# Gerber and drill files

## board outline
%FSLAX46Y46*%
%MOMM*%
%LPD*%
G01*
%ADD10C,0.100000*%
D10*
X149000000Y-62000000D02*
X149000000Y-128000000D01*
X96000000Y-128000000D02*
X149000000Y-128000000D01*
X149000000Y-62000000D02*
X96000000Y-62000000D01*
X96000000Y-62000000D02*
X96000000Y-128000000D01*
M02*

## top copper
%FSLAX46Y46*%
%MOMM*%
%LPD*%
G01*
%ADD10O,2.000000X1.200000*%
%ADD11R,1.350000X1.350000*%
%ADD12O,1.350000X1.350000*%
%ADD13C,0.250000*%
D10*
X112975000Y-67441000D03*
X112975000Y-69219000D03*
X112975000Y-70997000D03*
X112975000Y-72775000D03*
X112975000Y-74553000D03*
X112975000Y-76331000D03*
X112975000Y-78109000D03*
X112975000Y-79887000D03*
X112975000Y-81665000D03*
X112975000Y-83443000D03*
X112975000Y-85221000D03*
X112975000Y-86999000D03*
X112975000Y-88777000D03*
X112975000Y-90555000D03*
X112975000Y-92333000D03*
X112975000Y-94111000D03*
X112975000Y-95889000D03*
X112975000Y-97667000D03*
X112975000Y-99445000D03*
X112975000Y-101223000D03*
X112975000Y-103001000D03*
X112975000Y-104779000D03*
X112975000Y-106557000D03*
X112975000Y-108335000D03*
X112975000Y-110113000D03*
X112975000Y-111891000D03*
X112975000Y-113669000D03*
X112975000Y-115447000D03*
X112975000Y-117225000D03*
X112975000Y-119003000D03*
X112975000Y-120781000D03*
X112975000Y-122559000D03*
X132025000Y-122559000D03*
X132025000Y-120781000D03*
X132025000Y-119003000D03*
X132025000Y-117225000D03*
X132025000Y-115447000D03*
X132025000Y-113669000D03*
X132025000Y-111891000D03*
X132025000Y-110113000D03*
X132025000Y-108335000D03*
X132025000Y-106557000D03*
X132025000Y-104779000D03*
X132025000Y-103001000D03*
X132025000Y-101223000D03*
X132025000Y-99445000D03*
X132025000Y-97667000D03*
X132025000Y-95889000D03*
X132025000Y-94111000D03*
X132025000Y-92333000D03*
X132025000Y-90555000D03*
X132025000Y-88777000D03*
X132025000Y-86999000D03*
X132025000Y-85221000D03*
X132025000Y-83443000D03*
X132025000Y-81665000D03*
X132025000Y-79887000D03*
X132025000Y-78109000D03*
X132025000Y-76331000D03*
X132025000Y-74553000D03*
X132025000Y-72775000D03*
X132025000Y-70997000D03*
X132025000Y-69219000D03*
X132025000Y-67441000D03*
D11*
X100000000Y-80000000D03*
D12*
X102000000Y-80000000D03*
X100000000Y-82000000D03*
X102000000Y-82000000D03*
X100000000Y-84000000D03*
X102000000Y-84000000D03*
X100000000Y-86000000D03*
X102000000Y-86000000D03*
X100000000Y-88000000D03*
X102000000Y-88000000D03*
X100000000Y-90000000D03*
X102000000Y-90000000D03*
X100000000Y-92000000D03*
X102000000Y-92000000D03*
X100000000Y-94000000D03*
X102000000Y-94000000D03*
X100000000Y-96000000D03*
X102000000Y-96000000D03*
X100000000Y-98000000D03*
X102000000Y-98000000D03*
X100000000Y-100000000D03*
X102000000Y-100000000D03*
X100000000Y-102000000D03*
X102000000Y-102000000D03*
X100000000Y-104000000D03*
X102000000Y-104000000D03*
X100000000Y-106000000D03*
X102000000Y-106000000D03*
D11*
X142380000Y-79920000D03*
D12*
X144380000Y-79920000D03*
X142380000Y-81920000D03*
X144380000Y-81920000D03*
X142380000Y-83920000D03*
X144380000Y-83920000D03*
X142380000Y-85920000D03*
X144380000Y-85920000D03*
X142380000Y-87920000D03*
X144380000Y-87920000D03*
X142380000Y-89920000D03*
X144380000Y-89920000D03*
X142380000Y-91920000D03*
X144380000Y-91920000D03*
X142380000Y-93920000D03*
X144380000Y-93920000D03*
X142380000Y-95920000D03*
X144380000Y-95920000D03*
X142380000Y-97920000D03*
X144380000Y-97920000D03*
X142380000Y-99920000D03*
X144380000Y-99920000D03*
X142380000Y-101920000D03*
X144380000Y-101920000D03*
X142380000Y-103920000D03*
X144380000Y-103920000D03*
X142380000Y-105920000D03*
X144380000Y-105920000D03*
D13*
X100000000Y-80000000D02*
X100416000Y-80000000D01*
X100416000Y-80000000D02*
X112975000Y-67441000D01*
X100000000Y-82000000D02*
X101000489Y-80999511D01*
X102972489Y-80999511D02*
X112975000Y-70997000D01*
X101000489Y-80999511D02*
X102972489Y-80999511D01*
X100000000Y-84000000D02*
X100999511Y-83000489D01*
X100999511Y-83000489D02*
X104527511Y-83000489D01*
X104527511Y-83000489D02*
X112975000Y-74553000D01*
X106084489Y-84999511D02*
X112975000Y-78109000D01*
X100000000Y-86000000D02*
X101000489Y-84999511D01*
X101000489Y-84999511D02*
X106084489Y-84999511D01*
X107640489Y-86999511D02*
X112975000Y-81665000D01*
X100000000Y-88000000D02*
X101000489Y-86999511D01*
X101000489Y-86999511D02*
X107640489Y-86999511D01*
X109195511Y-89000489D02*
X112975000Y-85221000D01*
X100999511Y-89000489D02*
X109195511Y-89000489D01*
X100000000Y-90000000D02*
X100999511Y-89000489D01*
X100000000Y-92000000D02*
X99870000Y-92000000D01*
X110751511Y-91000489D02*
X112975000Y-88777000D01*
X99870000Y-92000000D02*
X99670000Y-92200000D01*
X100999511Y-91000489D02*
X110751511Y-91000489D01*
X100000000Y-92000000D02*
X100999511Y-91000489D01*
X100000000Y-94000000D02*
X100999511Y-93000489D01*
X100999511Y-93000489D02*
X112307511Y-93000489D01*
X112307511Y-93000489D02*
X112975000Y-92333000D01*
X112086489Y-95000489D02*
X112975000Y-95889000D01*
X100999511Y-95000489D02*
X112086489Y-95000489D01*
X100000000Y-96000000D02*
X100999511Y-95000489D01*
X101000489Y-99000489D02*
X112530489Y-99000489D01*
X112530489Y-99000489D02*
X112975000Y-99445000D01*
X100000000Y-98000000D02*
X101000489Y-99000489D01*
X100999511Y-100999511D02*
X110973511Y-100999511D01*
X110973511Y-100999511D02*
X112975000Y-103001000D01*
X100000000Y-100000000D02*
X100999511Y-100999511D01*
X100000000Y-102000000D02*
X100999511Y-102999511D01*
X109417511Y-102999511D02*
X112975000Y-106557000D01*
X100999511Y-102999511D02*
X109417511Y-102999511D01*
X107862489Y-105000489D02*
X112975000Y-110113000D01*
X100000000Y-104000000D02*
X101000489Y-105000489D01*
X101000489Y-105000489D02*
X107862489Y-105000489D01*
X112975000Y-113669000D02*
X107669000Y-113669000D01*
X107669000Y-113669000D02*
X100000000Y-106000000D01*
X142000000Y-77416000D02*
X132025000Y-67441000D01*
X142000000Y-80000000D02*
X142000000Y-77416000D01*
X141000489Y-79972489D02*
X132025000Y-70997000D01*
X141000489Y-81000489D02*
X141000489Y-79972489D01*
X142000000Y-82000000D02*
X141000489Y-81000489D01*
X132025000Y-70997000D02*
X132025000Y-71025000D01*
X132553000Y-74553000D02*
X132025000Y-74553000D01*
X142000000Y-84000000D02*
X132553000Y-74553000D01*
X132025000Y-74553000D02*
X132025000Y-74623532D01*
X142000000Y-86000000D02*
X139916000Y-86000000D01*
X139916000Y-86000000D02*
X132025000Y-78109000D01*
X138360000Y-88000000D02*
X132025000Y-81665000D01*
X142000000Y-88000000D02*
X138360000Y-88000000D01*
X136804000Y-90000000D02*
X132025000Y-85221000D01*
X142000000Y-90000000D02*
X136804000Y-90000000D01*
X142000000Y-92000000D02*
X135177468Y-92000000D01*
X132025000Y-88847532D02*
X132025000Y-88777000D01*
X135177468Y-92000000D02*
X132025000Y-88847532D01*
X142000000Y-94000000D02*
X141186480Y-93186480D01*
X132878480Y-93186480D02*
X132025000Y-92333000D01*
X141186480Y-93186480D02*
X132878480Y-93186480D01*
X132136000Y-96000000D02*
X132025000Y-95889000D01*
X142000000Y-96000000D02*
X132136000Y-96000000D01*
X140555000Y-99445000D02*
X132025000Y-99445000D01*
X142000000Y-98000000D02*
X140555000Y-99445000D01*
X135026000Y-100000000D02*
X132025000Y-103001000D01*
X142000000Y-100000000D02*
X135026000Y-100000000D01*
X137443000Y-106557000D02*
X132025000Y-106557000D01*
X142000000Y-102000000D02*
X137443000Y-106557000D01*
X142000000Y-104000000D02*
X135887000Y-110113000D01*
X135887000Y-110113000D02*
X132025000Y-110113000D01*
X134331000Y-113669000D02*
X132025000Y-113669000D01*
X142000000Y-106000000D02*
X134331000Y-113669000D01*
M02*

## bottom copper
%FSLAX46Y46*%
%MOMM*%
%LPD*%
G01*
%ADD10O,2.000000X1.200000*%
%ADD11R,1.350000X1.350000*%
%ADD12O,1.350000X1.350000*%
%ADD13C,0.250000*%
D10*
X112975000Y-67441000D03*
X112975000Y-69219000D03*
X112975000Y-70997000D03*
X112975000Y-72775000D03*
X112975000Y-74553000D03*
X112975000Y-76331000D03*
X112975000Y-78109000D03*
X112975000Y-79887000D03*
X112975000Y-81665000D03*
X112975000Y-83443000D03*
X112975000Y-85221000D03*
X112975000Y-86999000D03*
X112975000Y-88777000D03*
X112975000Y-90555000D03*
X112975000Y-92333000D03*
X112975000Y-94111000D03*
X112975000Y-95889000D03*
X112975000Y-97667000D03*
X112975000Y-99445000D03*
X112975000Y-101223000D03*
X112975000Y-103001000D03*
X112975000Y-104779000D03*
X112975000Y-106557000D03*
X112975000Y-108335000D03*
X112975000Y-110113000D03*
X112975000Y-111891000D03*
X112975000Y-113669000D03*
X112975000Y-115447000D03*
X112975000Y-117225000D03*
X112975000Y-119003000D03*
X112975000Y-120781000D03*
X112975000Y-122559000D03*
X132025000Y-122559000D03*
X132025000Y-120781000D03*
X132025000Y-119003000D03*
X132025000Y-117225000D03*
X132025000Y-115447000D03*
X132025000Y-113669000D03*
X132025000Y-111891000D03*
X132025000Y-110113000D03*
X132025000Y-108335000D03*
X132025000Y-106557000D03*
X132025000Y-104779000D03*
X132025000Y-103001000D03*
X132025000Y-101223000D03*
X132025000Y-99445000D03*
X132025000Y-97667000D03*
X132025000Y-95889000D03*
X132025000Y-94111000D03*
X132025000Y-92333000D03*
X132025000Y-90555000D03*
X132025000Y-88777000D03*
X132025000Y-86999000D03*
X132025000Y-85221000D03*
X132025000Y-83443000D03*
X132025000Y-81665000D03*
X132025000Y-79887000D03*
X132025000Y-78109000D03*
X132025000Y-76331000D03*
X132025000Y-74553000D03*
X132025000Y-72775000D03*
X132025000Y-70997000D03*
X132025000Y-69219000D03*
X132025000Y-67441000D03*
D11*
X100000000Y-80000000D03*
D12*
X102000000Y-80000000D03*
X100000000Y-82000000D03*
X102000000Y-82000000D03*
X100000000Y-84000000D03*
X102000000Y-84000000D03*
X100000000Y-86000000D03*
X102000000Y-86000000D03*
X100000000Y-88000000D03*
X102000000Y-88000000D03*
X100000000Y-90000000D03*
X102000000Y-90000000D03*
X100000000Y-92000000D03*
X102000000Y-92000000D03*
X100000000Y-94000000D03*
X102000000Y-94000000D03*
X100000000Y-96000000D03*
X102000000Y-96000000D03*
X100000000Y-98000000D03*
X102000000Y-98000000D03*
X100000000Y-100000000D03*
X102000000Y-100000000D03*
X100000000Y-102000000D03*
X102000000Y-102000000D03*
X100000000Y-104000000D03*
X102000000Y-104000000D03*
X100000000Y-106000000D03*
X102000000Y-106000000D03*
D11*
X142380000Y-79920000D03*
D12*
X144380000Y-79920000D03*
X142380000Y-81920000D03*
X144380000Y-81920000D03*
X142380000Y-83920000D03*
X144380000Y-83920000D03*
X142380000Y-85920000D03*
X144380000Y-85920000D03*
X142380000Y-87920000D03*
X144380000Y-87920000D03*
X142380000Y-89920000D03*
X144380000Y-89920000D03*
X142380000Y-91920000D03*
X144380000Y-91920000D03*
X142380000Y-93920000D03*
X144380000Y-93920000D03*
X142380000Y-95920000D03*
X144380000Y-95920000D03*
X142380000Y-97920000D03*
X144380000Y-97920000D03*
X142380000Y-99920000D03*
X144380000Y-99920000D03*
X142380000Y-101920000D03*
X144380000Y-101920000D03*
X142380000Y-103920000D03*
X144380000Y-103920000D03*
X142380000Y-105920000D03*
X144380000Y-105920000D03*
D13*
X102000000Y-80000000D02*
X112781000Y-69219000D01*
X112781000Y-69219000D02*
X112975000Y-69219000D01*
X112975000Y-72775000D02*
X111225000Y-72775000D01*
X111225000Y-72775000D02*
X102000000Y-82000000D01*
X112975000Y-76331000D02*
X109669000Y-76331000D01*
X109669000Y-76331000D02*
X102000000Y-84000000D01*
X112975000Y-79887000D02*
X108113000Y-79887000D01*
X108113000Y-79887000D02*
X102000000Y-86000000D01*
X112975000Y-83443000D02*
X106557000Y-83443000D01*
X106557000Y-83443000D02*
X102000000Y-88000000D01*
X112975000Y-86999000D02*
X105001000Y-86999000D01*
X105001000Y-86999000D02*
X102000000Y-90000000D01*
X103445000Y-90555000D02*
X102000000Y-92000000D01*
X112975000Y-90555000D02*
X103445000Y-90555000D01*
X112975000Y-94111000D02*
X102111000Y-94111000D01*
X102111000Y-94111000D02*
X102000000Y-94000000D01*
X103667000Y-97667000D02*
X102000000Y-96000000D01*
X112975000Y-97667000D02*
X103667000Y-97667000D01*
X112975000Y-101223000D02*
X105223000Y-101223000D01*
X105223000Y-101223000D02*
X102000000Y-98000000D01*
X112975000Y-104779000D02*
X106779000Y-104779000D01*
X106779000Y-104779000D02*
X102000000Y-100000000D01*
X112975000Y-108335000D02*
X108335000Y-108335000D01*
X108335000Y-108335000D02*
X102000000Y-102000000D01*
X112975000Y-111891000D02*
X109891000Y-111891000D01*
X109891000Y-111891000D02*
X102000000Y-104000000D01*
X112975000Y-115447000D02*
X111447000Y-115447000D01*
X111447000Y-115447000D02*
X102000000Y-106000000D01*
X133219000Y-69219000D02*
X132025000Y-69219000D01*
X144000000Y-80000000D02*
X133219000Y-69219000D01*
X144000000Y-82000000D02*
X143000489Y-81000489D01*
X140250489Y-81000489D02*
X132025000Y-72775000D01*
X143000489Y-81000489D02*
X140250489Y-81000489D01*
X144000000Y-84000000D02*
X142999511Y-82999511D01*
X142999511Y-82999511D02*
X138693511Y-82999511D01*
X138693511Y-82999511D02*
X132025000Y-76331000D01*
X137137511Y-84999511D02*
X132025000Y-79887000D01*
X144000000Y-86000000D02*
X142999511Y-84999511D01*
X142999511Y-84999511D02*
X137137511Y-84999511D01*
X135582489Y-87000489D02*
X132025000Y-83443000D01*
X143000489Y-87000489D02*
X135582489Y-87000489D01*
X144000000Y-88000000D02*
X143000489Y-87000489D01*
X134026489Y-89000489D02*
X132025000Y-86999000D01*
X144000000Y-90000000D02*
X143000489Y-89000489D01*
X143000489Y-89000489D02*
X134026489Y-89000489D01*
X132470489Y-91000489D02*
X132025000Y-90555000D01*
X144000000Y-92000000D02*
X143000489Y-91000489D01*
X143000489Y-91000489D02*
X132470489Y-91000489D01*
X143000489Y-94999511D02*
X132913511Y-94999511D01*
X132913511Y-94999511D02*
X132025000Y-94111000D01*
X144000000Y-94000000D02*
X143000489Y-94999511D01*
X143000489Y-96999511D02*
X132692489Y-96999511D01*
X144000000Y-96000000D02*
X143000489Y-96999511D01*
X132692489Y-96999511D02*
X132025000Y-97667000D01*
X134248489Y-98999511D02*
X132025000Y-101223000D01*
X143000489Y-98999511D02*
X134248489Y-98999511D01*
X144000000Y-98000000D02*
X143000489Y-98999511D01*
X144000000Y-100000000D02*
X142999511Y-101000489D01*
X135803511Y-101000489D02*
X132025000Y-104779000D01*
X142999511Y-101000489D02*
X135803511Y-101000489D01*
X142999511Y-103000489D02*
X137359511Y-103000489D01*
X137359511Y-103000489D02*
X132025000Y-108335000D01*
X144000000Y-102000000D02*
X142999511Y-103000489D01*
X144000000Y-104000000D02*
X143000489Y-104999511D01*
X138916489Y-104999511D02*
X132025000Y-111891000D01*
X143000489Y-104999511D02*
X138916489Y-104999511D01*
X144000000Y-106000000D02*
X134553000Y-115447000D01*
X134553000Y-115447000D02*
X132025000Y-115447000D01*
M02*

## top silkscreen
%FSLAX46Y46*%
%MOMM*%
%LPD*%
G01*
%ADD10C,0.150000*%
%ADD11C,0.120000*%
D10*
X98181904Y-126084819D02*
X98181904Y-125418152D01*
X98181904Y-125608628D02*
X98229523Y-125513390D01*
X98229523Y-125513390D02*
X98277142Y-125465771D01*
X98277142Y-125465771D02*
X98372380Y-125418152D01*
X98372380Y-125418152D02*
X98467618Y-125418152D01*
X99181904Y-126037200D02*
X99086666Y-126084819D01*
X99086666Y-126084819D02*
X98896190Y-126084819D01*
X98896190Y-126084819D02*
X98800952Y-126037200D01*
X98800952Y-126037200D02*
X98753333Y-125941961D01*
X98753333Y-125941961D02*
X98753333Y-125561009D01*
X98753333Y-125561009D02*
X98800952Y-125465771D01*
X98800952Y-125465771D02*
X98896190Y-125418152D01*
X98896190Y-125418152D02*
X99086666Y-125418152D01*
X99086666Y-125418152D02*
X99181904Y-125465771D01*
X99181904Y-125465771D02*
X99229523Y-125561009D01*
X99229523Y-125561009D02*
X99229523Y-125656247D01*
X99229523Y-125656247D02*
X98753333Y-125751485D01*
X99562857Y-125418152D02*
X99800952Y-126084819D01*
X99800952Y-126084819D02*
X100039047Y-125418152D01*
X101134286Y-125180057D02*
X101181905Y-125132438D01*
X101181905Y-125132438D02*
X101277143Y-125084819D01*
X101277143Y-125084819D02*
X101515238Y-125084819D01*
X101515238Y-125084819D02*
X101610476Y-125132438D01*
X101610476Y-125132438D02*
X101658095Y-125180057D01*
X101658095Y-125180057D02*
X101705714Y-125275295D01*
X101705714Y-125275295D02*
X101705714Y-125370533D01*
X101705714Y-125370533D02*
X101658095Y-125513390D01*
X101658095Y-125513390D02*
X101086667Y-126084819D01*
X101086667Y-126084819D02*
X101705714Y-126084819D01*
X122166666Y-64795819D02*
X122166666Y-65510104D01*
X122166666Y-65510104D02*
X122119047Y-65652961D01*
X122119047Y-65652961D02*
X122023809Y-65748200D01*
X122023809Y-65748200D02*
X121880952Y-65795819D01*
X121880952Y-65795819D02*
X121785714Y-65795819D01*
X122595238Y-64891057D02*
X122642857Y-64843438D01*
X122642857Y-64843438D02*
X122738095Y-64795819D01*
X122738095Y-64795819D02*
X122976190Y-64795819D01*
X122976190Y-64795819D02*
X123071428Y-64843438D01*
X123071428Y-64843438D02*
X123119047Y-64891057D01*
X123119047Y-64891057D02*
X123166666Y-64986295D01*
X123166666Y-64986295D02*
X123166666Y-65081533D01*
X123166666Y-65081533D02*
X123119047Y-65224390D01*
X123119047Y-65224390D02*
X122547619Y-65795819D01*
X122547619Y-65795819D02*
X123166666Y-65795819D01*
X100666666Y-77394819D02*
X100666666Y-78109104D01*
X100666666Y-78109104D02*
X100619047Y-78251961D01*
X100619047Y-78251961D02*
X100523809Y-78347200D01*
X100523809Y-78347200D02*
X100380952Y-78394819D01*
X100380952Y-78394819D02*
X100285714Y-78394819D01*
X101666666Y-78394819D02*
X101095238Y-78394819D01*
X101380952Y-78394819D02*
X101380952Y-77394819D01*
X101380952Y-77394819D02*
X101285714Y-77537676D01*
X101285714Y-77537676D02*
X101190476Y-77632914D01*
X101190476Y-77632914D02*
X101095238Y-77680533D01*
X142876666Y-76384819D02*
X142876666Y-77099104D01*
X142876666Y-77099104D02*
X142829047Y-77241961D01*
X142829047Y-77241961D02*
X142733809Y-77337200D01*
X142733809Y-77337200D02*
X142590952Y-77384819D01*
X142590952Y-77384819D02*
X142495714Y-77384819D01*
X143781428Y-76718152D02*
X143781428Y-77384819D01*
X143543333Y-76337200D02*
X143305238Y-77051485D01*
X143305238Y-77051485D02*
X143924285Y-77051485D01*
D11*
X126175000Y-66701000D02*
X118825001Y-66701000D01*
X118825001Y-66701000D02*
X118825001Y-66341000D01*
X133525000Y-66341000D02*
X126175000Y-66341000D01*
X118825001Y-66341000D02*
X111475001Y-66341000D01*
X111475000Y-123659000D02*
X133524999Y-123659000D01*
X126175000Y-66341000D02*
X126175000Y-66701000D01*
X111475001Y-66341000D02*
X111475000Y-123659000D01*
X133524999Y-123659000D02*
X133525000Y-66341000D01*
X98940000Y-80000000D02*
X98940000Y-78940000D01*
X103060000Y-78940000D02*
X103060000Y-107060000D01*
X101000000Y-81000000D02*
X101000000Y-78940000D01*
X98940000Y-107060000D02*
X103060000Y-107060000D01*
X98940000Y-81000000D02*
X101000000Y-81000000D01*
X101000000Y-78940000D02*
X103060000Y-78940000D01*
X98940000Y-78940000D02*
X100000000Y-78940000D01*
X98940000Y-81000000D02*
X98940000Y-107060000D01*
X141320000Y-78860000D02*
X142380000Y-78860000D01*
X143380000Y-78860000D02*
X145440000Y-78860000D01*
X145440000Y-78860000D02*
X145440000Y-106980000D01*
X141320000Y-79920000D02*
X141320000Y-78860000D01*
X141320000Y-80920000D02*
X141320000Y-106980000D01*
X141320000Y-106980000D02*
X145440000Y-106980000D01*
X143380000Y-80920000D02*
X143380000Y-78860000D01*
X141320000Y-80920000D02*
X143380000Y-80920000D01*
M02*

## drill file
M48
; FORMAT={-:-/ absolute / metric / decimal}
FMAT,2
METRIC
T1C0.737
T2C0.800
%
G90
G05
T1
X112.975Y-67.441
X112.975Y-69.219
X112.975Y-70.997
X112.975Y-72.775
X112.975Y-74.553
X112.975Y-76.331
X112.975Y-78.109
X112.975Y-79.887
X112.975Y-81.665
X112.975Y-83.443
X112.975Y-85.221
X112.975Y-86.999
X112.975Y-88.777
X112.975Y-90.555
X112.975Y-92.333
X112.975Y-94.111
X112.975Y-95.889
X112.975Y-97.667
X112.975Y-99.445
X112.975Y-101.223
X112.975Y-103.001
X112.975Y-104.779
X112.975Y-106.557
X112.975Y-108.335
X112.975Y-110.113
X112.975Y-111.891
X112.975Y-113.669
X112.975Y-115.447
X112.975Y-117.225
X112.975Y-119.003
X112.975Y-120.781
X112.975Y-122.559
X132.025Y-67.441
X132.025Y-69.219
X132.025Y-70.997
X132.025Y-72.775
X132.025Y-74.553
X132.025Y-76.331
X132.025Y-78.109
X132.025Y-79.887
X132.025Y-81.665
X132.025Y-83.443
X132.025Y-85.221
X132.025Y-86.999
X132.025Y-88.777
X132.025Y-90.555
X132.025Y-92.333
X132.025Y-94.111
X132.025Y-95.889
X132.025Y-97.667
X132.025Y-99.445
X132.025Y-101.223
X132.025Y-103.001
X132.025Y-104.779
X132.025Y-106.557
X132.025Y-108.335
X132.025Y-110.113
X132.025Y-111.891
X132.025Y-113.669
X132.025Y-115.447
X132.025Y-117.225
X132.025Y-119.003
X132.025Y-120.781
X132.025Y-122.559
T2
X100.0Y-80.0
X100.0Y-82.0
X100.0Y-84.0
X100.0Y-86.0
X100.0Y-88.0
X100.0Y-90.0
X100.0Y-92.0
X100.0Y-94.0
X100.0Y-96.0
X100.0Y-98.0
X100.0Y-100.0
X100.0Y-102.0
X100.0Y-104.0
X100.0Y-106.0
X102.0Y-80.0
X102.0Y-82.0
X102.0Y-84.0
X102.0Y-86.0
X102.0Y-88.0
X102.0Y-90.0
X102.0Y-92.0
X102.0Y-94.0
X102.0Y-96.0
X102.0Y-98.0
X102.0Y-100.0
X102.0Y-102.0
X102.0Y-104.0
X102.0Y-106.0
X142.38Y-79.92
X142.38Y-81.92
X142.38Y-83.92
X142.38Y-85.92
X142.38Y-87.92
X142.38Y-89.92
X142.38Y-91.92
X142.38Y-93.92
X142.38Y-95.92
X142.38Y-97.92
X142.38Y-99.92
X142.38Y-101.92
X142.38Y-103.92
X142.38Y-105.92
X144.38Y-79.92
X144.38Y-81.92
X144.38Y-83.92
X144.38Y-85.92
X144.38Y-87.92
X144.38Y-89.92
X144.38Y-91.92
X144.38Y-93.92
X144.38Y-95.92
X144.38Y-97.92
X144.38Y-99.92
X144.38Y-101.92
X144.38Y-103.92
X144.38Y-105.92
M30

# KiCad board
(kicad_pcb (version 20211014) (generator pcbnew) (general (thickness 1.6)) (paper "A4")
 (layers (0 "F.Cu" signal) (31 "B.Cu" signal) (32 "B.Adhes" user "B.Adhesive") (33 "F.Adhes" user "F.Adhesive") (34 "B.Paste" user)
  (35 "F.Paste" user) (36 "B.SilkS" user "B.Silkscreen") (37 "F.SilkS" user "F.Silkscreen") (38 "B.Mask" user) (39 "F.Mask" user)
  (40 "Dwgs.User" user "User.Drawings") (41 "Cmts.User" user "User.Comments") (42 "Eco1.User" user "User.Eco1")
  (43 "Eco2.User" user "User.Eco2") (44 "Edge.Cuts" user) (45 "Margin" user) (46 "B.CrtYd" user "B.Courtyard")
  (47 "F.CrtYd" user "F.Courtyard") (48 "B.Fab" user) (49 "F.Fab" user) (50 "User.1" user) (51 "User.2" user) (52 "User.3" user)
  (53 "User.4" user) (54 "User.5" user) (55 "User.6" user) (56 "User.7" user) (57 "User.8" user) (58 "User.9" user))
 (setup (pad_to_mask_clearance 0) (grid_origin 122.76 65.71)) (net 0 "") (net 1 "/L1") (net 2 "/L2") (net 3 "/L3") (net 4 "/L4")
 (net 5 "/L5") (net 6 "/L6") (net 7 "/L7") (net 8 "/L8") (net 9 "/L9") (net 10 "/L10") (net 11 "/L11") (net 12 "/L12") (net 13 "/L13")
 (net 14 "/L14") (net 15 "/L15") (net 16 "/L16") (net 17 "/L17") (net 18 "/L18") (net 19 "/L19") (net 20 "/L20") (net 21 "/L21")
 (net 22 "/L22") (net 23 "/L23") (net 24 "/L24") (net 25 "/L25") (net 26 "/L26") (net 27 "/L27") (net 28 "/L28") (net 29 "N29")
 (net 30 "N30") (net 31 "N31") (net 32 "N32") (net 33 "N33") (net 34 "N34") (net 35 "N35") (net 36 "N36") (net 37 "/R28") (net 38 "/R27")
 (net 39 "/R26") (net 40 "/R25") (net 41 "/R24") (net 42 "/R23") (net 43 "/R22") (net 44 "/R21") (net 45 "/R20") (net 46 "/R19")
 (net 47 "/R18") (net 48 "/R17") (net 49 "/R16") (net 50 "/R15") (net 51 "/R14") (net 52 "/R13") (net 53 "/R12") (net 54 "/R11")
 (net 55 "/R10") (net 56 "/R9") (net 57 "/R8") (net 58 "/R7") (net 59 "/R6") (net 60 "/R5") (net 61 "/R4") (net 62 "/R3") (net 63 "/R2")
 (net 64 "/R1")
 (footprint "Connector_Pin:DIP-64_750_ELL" (layer "F.Cu") (at 122.5 95)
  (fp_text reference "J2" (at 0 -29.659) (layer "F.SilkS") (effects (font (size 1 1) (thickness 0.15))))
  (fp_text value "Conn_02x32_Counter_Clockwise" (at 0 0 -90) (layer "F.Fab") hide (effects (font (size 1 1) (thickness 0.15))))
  (fp_line (start 3.675 -28.299) (end -3.674999 -28.299) (layer "F.SilkS") (width 0.12))
  (fp_line (start -3.674999 -28.299) (end -3.674999 -28.659) (layer "F.SilkS") (width 0.12))
  (fp_line (start 11.025 -28.659) (end 3.675 -28.659) (layer "F.SilkS") (width 0.12))
  (fp_line (start -3.674999 -28.659) (end -11.024999 -28.659) (layer "F.SilkS") (width 0.12))
  (fp_line (start -11.025 28.659) (end 11.024999 28.659) (layer "F.SilkS") (width 0.12))
  (fp_line (start 3.675 -28.659) (end 3.675 -28.299) (layer "F.SilkS") (width 0.12))
  (fp_line (start -11.024999 -28.659) (end -11.025 28.659) (layer "F.SilkS") (width 0.12))
  (fp_line (start 11.024999 28.659) (end 11.025 -28.659) (layer "F.SilkS") (width 0.12))
  (pad "1" thru_hole oval (at -9.525 -27.559 270) (size 1.2 2) (drill 0.7366) (layers *.Cu *.Mask) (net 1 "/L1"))
  (pad "2" thru_hole oval (at -9.525 -25.781 270) (size 1.2 2) (drill 0.7366) (layers *.Cu *.Mask) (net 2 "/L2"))
  (pad "3" thru_hole oval (at -9.525 -24.003 270) (size 1.2 2) (drill 0.7366) (layers *.Cu *.Mask) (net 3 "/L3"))
  (pad "4" thru_hole oval (at -9.525 -22.225 270) (size 1.2 2) (drill 0.7366) (layers *.Cu *.Mask) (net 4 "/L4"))
  (pad "5" thru_hole oval (at -9.525 -20.447 270) (size 1.2 2) (drill 0.7366) (layers *.Cu *.Mask) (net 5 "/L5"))
  (pad "6" thru_hole oval (at -9.525 -18.669 270) (size 1.2 2) (drill 0.7366) (layers *.Cu *.Mask) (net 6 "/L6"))
  (pad "7" thru_hole oval (at -9.525 -16.891 270) (size 1.2 2) (drill 0.7366) (layers *.Cu *.Mask) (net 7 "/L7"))
  (pad "8" thru_hole oval (at -9.525 -15.113 270) (size 1.2 2) (drill 0.7366) (layers *.Cu *.Mask) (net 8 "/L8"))
  (pad "9" thru_hole oval (at -9.525 -13.335 270) (size 1.2 2) (drill 0.7366) (layers *.Cu *.Mask) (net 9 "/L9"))
  (pad "10" thru_hole oval (at -9.525 -11.557 270) (size 1.2 2) (drill 0.7366) (layers *.Cu *.Mask) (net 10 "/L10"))
  (pad "11" thru_hole oval (at -9.525 -9.779 270) (size 1.2 2) (drill 0.7366) (layers *.Cu *.Mask) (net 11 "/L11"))
  (pad "12" thru_hole oval (at -9.525 -8.001 270) (size 1.2 2) (drill 0.7366) (layers *.Cu *.Mask) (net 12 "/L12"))
  (pad "13" thru_hole oval (at -9.525 -6.223 270) (size 1.2 2) (drill 0.7366) (layers *.Cu *.Mask) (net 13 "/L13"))
  (pad "14" thru_hole oval (at -9.525 -4.445 270) (size 1.2 2) (drill 0.7366) (layers *.Cu *.Mask) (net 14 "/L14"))
  (pad "15" thru_hole oval (at -9.525 -2.667 270) (size 1.2 2) (drill 0.7366) (layers *.Cu *.Mask) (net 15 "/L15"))
  (pad "16" thru_hole oval (at -9.525 -0.889 270) (size 1.2 2) (drill 0.7366) (layers *.Cu *.Mask) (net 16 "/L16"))
  (pad "17" thru_hole oval (at -9.525 0.889 270) (size 1.2 2) (drill 0.7366) (layers *.Cu *.Mask) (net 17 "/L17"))
  (pad "18" thru_hole oval (at -9.525 2.667 270) (size 1.2 2) (drill 0.7366) (layers *.Cu *.Mask) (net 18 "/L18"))
  (pad "19" thru_hole oval (at -9.525 4.445 270) (size 1.2 2) (drill 0.7366) (layers *.Cu *.Mask) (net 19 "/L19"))
  (pad "20" thru_hole oval (at -9.525 6.223 270) (size 1.2 2) (drill 0.7366) (layers *.Cu *.Mask) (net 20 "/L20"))
  (pad "21" thru_hole oval (at -9.525 8.001 270) (size 1.2 2) (drill 0.7366) (layers *.Cu *.Mask) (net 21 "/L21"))
  (pad "22" thru_hole oval (at -9.525 9.779 270) (size 1.2 2) (drill 0.7366) (layers *.Cu *.Mask) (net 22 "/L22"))
  (pad "23" thru_hole oval (at -9.525 11.557 270) (size 1.2 2) (drill 0.7366) (layers *.Cu *.Mask) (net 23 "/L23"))
  (pad "24" thru_hole oval (at -9.525 13.335 270) (size 1.2 2) (drill 0.7366) (layers *.Cu *.Mask) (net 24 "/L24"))
  (pad "25" thru_hole oval (at -9.525 15.113 270) (size 1.2 2) (drill 0.7366) (layers *.Cu *.Mask) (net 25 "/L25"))
  (pad "26" thru_hole oval (at -9.525 16.891 270) (size 1.2 2) (drill 0.7366) (layers *.Cu *.Mask) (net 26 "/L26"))
  (pad "27" thru_hole oval (at -9.525 18.669 270) (size 1.2 2) (drill 0.7366) (layers *.Cu *.Mask) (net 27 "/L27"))
  (pad "28" thru_hole oval (at -9.525 20.447 270) (size 1.2 2) (drill 0.7366) (layers *.Cu *.Mask) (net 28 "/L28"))
  (pad "29" thru_hole oval (at -9.525 22.225 270) (size 1.2 2) (drill 0.7366) (layers *.Cu *.Mask) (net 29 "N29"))
  (pad "30" thru_hole oval (at -9.525 24.003 270) (size 1.2 2) (drill 0.7366) (layers *.Cu *.Mask) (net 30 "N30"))
  (pad "31" thru_hole oval (at -9.525 25.781 270) (size 1.2 2) (drill 0.7366) (layers *.Cu *.Mask) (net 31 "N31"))
  (pad "32" thru_hole oval (at -9.525 27.559 270) (size 1.2 2) (drill 0.7366) (layers *.Cu *.Mask) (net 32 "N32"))
  (pad "33" thru_hole oval (at 9.525 27.559 270) (size 1.2 2) (drill 0.7366) (layers *.Cu *.Mask) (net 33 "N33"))
  (pad "34" thru_hole oval (at 9.525 25.781 270) (size 1.2 2) (drill 0.7366) (layers *.Cu *.Mask) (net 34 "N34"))
  (pad "35" thru_hole oval (at 9.525 24.003 270) (size 1.2 2) (drill 0.7366) (layers *.Cu *.Mask) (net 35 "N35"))
  (pad "36" thru_hole oval (at 9.525 22.225 270) (size 1.2 2) (drill 0.7366) (layers *.Cu *.Mask) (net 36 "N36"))
  (pad "37" thru_hole oval (at 9.525 20.447 270) (size 1.2 2) (drill 0.7366) (layers *.Cu *.Mask) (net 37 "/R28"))
  (pad "38" thru_hole oval (at 9.525 18.669 270) (size 1.2 2) (drill 0.7366) (layers *.Cu *.Mask) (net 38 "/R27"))
  (pad "39" thru_hole oval (at 9.525 16.891 270) (size 1.2 2) (drill 0.7366) (layers *.Cu *.Mask) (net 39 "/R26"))
  (pad "40" thru_hole oval (at 9.525 15.113 270) (size 1.2 2) (drill 0.7366) (layers *.Cu *.Mask) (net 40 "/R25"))
  (pad "41" thru_hole oval (at 9.525 13.335 270) (size 1.2 2) (drill 0.7366) (layers *.Cu *.Mask) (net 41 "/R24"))
  (pad "42" thru_hole oval (at 9.525 11.557 270) (size 1.2 2) (drill 0.7366) (layers *.Cu *.Mask) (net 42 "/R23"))
  (pad "43" thru_hole oval (at 9.525 9.779 270) (size 1.2 2) (drill 0.7366) (layers *.Cu *.Mask) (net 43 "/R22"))
  (pad "44" thru_hole oval (at 9.525 8.001 270) (size 1.2 2) (drill 0.7366) (layers *.Cu *.Mask) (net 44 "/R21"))
  (pad "45" thru_hole oval (at 9.525 6.223 270) (size 1.2 2) (drill 0.7366) (layers *.Cu *.Mask) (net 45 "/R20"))
  (pad "46" thru_hole oval (at 9.525 4.445 270) (size 1.2 2) (drill 0.7366) (layers *.Cu *.Mask) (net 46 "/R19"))
  (pad "47" thru_hole oval (at 9.525 2.667 270) (size 1.2 2) (drill 0.7366) (layers *.Cu *.Mask) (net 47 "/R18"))
  (pad "48" thru_hole oval (at 9.525 0.889 270) (size 1.2 2) (drill 0.7366) (layers *.Cu *.Mask) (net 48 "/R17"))
  (pad "49" thru_hole oval (at 9.525 -0.889 270) (size 1.2 2) (drill 0.7366) (layers *.Cu *.Mask) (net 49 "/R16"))
  (pad "50" thru_hole oval (at 9.525 -2.667 270) (size 1.2 2) (drill 0.7366) (layers *.Cu *.Mask) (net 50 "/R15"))
  (pad "51" thru_hole oval (at 9.525 -4.445 270) (size 1.2 2) (drill 0.7366) (layers *.Cu *.Mask) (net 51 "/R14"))
  (pad "52" thru_hole oval (at 9.525 -6.223 270) (size 1.2 2) (drill 0.7366) (layers *.Cu *.Mask) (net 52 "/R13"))
  (pad "53" thru_hole oval (at 9.525 -8.001 270) (size 1.2 2) (drill 0.7366) (layers *.Cu *.Mask) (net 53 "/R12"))
  (pad "54" thru_hole oval (at 9.525 -9.779 270) (size 1.2 2) (drill 0.7366) (layers *.Cu *.Mask) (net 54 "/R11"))
  (pad "55" thru_hole oval (at 9.525 -11.557 270) (size 1.2 2) (drill 0.7366) (layers *.Cu *.Mask) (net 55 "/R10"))
  (pad "56" thru_hole oval (at 9.525 -13.335 270) (size 1.2 2) (drill 0.7366) (layers *.Cu *.Mask) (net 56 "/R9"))
  (pad "57" thru_hole oval (at 9.525 -15.113 270) (size 1.2 2) (drill 0.7366) (layers *.Cu *.Mask) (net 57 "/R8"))
  (pad "58" thru_hole oval (at 9.525 -16.891 270) (size 1.2 2) (drill 0.7366) (layers *.Cu *.Mask) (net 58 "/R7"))
  (pad "59" thru_hole oval (at 9.525 -18.669 270) (size 1.2 2) (drill 0.7366) (layers *.Cu *.Mask) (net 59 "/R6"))
  (pad "60" thru_hole oval (at 9.525 -20.447 270) (size 1.2 2) (drill 0.7366) (layers *.Cu *.Mask) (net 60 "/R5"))
  (pad "61" thru_hole oval (at 9.525 -22.225 270) (size 1.2 2) (drill 0.7366) (layers *.Cu *.Mask) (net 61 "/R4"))
  (pad "62" thru_hole oval (at 9.525 -24.003 270) (size 1.2 2) (drill 0.7366) (layers *.Cu *.Mask) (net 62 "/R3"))
  (pad "63" thru_hole oval (at 9.525 -25.781 270) (size 1.2 2) (drill 0.7366) (layers *.Cu *.Mask) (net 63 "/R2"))
  (pad "64" thru_hole oval (at 9.525 -27.559 270) (size 1.2 2) (drill 0.7366) (layers *.Cu *.Mask) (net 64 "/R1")))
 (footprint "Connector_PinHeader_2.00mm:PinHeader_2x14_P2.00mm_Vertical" (layer "F.Cu") (at 100 80)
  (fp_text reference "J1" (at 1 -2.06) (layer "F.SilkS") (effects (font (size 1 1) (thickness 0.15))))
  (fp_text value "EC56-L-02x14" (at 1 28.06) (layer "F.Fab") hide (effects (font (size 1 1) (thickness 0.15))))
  (fp_line (start -1.06 0) (end -1.06 -1.06) (layer "F.SilkS") (width 0.12))
  (fp_line (start 3.06 -1.06) (end 3.06 27.06) (layer "F.SilkS") (width 0.12))
  (fp_line (start 1 1) (end 1 -1.06) (layer "F.SilkS") (width 0.12))
  (fp_line (start -1.06 27.06) (end 3.06 27.06) (layer "F.SilkS") (width 0.12))
  (fp_line (start -1.06 1) (end 1 1) (layer "F.SilkS") (width 0.12))
  (fp_line (start 1 -1.06) (end 3.06 -1.06) (layer "F.SilkS") (width 0.12))
  (fp_line (start -1.06 -1.06) (end 0 -1.06) (layer "F.SilkS") (width 0.12))
  (fp_line (start -1.06 1) (end -1.06 27.06) (layer "F.SilkS") (width 0.12))
  (pad "1" thru_hole rect locked (at 0 0) (size 1.35 1.35) (drill 0.8) (layers *.Cu *.Mask) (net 1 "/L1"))
  (pad "2" thru_hole oval locked (at 2 0) (size 1.35 1.35) (drill 0.8) (layers *.Cu *.Mask) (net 2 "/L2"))
  (pad "3" thru_hole oval locked (at 0 2) (size 1.35 1.35) (drill 0.8) (layers *.Cu *.Mask) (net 3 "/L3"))
  (pad "4" thru_hole oval locked (at 2 2) (size 1.35 1.35) (drill 0.8) (layers *.Cu *.Mask) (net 4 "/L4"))
  (pad "5" thru_hole oval locked (at 0 4) (size 1.35 1.35) (drill 0.8) (layers *.Cu *.Mask) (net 5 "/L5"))
  (pad "6" thru_hole oval locked (at 2 4) (size 1.35 1.35) (drill 0.8) (layers *.Cu *.Mask) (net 6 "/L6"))
  (pad "7" thru_hole oval locked (at 0 6) (size 1.35 1.35) (drill 0.8) (layers *.Cu *.Mask) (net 7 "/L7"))
  (pad "8" thru_hole oval locked (at 2 6) (size 1.35 1.35) (drill 0.8) (layers *.Cu *.Mask) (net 8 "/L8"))
  (pad "9" thru_hole oval locked (at 0 8) (size 1.35 1.35) (drill 0.8) (layers *.Cu *.Mask) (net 9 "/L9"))
  (pad "10" thru_hole oval locked (at 2 8) (size 1.35 1.35) (drill 0.8) (layers *.Cu *.Mask) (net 10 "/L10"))
  (pad "11" thru_hole oval locked (at 0 10) (size 1.35 1.35) (drill 0.8) (layers *.Cu *.Mask) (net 11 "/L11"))
  (pad "12" thru_hole oval locked (at 2 10) (size 1.35 1.35) (drill 0.8) (layers *.Cu *.Mask) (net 12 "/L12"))
  (pad "13" thru_hole oval locked (at 0 12) (size 1.35 1.35) (drill 0.8) (layers *.Cu *.Mask) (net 13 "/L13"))
  (pad "14" thru_hole oval locked (at 2 12) (size 1.35 1.35) (drill 0.8) (layers *.Cu *.Mask) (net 14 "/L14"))
  (pad "15" thru_hole oval locked (at 0 14) (size 1.35 1.35) (drill 0.8) (layers *.Cu *.Mask) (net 15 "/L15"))
  (pad "16" thru_hole oval locked (at 2 14) (size 1.35 1.35) (drill 0.8) (layers *.Cu *.Mask) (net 16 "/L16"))
  (pad "17" thru_hole oval locked (at 0 16) (size 1.35 1.35) (drill 0.8) (layers *.Cu *.Mask) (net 17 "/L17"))
  (pad "18" thru_hole oval locked (at 2 16) (size 1.35 1.35) (drill 0.8) (layers *.Cu *.Mask) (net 18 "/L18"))
  (pad "19" thru_hole oval locked (at 0 18) (size 1.35 1.35) (drill 0.8) (layers *.Cu *.Mask) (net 19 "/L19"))
  (pad "20" thru_hole oval locked (at 2 18) (size 1.35 1.35) (drill 0.8) (layers *.Cu *.Mask) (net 20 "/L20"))
  (pad "21" thru_hole oval locked (at 0 20) (size 1.35 1.35) (drill 0.8) (layers *.Cu *.Mask) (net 21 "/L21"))
  (pad "22" thru_hole oval locked (at 2 20) (size 1.35 1.35) (drill 0.8) (layers *.Cu *.Mask) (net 22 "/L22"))
  (pad "23" thru_hole oval locked (at 0 22) (size 1.35 1.35) (drill 0.8) (layers *.Cu *.Mask) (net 23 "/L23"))
  (pad "24" thru_hole oval locked (at 2 22) (size 1.35 1.35) (drill 0.8) (layers *.Cu *.Mask) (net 24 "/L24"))
  (pad "25" thru_hole oval locked (at 0 24) (size 1.35 1.35) (drill 0.8) (layers *.Cu *.Mask) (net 25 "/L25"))
  (pad "26" thru_hole oval locked (at 2 24) (size 1.35 1.35) (drill 0.8) (layers *.Cu *.Mask) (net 26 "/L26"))
  (pad "27" thru_hole oval locked (at 0 26) (size 1.35 1.35) (drill 0.8) (layers *.Cu *.Mask) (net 27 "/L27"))
  (pad "28" thru_hole oval locked (at 2 26) (size 1.35 1.35) (drill 0.8) (layers *.Cu *.Mask) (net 28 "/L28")))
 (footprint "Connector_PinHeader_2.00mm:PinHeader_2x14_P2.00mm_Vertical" (layer "F.Cu") (at 142.38 79.92)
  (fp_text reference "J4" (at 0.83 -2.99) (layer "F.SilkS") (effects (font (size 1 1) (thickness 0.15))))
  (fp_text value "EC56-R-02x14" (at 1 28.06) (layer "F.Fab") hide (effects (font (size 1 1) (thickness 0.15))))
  (fp_line (start -1.06 -1.06) (end 0 -1.06) (layer "F.SilkS") (width 0.12))
  (fp_line (start 1 -1.06) (end 3.06 -1.06) (layer "F.SilkS") (width 0.12))
  (fp_line (start 3.06 -1.06) (end 3.06 27.06) (layer "F.SilkS") (width 0.12))
  (fp_line (start -1.06 0) (end -1.06 -1.06) (layer "F.SilkS") (width 0.12))
  (fp_line (start -1.06 1) (end -1.06 27.06) (layer "F.SilkS") (width 0.12))
  (fp_line (start -1.06 27.06) (end 3.06 27.06) (layer "F.SilkS") (width 0.12))
  (fp_line (start 1 1) (end 1 -1.06) (layer "F.SilkS") (width 0.12))
  (fp_line (start -1.06 1) (end 1 1) (layer "F.SilkS") (width 0.12))
  (pad "1" thru_hole rect locked (at 0 0) (size 1.35 1.35) (drill 0.8) (layers *.Cu *.Mask) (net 64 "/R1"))
  (pad "2" thru_hole oval locked (at 2 0) (size 1.35 1.35) (drill 0.8) (layers *.Cu *.Mask) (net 63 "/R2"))
  (pad "3" thru_hole oval locked (at 0 2) (size 1.35 1.35) (drill 0.8) (layers *.Cu *.Mask) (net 62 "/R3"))
  (pad "4" thru_hole oval locked (at 2 2) (size 1.35 1.35) (drill 0.8) (layers *.Cu *.Mask) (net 61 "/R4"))
  (pad "5" thru_hole oval locked (at 0 4) (size 1.35 1.35) (drill 0.8) (layers *.Cu *.Mask) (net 60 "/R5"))
  (pad "6" thru_hole oval locked (at 2 4) (size 1.35 1.35) (drill 0.8) (layers *.Cu *.Mask) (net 59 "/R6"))
  (pad "7" thru_hole oval locked (at 0 6) (size 1.35 1.35) (drill 0.8) (layers *.Cu *.Mask) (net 58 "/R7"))
  (pad "8" thru_hole oval locked (at 2 6) (size 1.35 1.35) (drill 0.8) (layers *.Cu *.Mask) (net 57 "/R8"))
  (pad "9" thru_hole oval locked (at 0 8) (size 1.35 1.35) (drill 0.8) (layers *.Cu *.Mask) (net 56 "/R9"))
  (pad "10" thru_hole oval locked (at 2 8) (size 1.35 1.35) (drill 0.8) (layers *.Cu *.Mask) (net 55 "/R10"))
  (pad "11" thru_hole oval locked (at 0 10) (size 1.35 1.35) (drill 0.8) (layers *.Cu *.Mask) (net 54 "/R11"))
  (pad "12" thru_hole oval locked (at 2 10) (size 1.35 1.35) (drill 0.8) (layers *.Cu *.Mask) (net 53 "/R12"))
  (pad "13" thru_hole oval locked (at 0 12) (size 1.35 1.35) (drill 0.8) (layers *.Cu *.Mask) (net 52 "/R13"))
  (pad "14" thru_hole oval locked (at 2 12) (size 1.35 1.35) (drill 0.8) (layers *.Cu *.Mask) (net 51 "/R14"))
  (pad "15" thru_hole oval locked (at 0 14) (size 1.35 1.35) (drill 0.8) (layers *.Cu *.Mask) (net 50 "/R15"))
  (pad "16" thru_hole oval locked (at 2 14) (size 1.35 1.35) (drill 0.8) (layers *.Cu *.Mask) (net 49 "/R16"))
  (pad "17" thru_hole oval locked (at 0 16) (size 1.35 1.35) (drill 0.8) (layers *.Cu *.Mask) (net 48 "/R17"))
  (pad "18" thru_hole oval locked (at 2 16) (size 1.35 1.35) (drill 0.8) (layers *.Cu *.Mask) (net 47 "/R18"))
  (pad "19" thru_hole oval locked (at 0 18) (size 1.35 1.35) (drill 0.8) (layers *.Cu *.Mask) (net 46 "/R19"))
  (pad "20" thru_hole oval locked (at 2 18) (size 1.35 1.35) (drill 0.8) (layers *.Cu *.Mask) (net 45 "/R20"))
  (pad "21" thru_hole oval locked (at 0 20) (size 1.35 1.35) (drill 0.8) (layers *.Cu *.Mask) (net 44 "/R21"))
  (pad "22" thru_hole oval locked (at 2 20) (size 1.35 1.35) (drill 0.8) (layers *.Cu *.Mask) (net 43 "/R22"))
  (pad "23" thru_hole oval locked (at 0 22) (size 1.35 1.35) (drill 0.8) (layers *.Cu *.Mask) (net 42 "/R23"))
  (pad "24" thru_hole oval locked (at 2 22) (size 1.35 1.35) (drill 0.8) (layers *.Cu *.Mask) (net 41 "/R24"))
  (pad "25" thru_hole oval locked (at 0 24) (size 1.35 1.35) (drill 0.8) (layers *.Cu *.Mask) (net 40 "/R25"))
  (pad "26" thru_hole oval locked (at 2 24) (size 1.35 1.35) (drill 0.8) (layers *.Cu *.Mask) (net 39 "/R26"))
  (pad "27" thru_hole oval locked (at 0 26) (size 1.35 1.35) (drill 0.8) (layers *.Cu *.Mask) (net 38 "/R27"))
  (pad "28" thru_hole oval locked (at 2 26) (size 1.35 1.35) (drill 0.8) (layers *.Cu *.Mask) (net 37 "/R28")))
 (gr_line (start 149 62) (end 149 128) (layer "Edge.Cuts") (width 0.1))
 (gr_line (start 96 128) (end 149 128) (layer "Edge.Cuts") (width 0.1))
 (gr_line (start 149 62) (end 96 62) (layer "Edge.Cuts") (width 0.1))
 (gr_line (start 96 62) (end 96 128) (layer "Edge.Cuts") (width 0.1))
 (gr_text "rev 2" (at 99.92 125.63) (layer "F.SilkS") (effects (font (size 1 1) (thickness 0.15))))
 (segment (start 100 80) (end 100.416 80) (width 0.25) (layer "F.Cu") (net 1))
 (segment (start 100.416 80) (end 112.975 67.441) (width 0.25) (layer "F.Cu") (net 1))
 (segment (start 102 80) (end 112.781 69.219) (width 0.25) (layer "B.Cu") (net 2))
 (segment (start 112.781 69.219) (end 112.975 69.219) (width 0.25) (layer "B.Cu") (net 2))
 (segment (start 100 82) (end 101.000489 80.999511) (width 0.25) (layer "F.Cu") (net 3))
 (segment (start 102.972489 80.999511) (end 112.975 70.997) (width 0.25) (layer "F.Cu") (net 3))
 (segment (start 101.000489 80.999511) (end 102.972489 80.999511) (width 0.25) (layer "F.Cu") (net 3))
 (segment (start 112.975 72.775) (end 111.225 72.775) (width 0.25) (layer "B.Cu") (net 4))
 (segment (start 111.225 72.775) (end 102 82) (width 0.25) (layer "B.Cu") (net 4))
 (segment (start 100 84) (end 100.999511 83.000489) (width 0.25) (layer "F.Cu") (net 5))
 (segment (start 100.999511 83.000489) (end 104.527511 83.000489) (width 0.25) (layer "F.Cu") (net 5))
 (segment (start 104.527511 83.000489) (end 112.975 74.553) (width 0.25) (layer "F.Cu") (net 5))
 (segment (start 112.975 76.331) (end 109.669 76.331) (width 0.25) (layer "B.Cu") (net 6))
 (segment (start 109.669 76.331) (end 102 84) (width 0.25) (layer "B.Cu") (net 6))
 (segment (start 106.084489 84.999511) (end 112.975 78.109) (width 0.25) (layer "F.Cu") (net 7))
 (segment (start 100 86) (end 101.000489 84.999511) (width 0.25) (layer "F.Cu") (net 7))
 (segment (start 101.000489 84.999511) (end 106.084489 84.999511) (width 0.25) (layer "F.Cu") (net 7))
 (segment (start 112.975 79.887) (end 108.113 79.887) (width 0.25) (layer "B.Cu") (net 8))
 (segment (start 108.113 79.887) (end 102 86) (width 0.25) (layer "B.Cu") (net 8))
 (segment (start 107.640489 86.999511) (end 112.975 81.665) (width 0.25) (layer "F.Cu") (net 9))
 (segment (start 100 88) (end 101.000489 86.999511) (width 0.25) (layer "F.Cu") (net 9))
 (segment (start 101.000489 86.999511) (end 107.640489 86.999511) (width 0.25) (layer "F.Cu") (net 9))
 (segment (start 112.975 83.443) (end 106.557 83.443) (width 0.25) (layer "B.Cu") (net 10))
 (segment (start 106.557 83.443) (end 102 88) (width 0.25) (layer "B.Cu") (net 10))
 (segment (start 109.195511 89.000489) (end 112.975 85.221) (width 0.25) (layer "F.Cu") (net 11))
 (segment (start 100.999511 89.000489) (end 109.195511 89.000489) (width 0.25) (layer "F.Cu") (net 11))
 (segment (start 100 90) (end 100.999511 89.000489) (width 0.25) (layer "F.Cu") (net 11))
 (segment (start 112.975 86.999) (end 105.001 86.999) (width 0.25) (layer "B.Cu") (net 12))
 (segment (start 105.001 86.999) (end 102 90) (width 0.25) (layer "B.Cu") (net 12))
 (segment (start 100 92) (end 99.87 92) (width 0.25) (layer "F.Cu") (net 13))
 (segment (start 110.751511 91.000489) (end 112.975 88.777) (width 0.25) (layer "F.Cu") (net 13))
 (segment (start 99.87 92) (end 99.67 92.2) (width 0.25) (layer "F.Cu") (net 13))
 (segment (start 100.999511 91.000489) (end 110.751511 91.000489) (width 0.25) (layer "F.Cu") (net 13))
 (segment (start 100 92) (end 100.999511 91.000489) (width 0.25) (layer "F.Cu") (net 13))
 (segment (start 103.445 90.555) (end 102 92) (width 0.25) (layer "B.Cu") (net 14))
 (segment (start 112.975 90.555) (end 103.445 90.555) (width 0.25) (layer "B.Cu") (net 14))
 (segment (start 100 94) (end 100.999511 93.000489) (width 0.25) (layer "F.Cu") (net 15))
 (segment (start 100.999511 93.000489) (end 112.307511 93.000489) (width 0.25) (layer "F.Cu") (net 15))
 (segment (start 112.307511 93.000489) (end 112.975 92.333) (width 0.25) (layer "F.Cu") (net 15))
 (segment (start 112.975 94.111) (end 102.111 94.111) (width 0.25) (layer "B.Cu") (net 16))
 (segment (start 102.111 94.111) (end 102 94) (width 0.25) (layer "B.Cu") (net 16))
 (segment (start 112.086489 95.000489) (end 112.975 95.889) (width 0.25) (layer "F.Cu") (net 17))
 (segment (start 100.999511 95.000489) (end 112.086489 95.000489) (width 0.25) (layer "F.Cu") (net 17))
 (segment (start 100 96) (end 100.999511 95.000489) (width 0.25) (layer "F.Cu") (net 17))
 (segment (start 103.667 97.667) (end 102 96) (width 0.25) (layer "B.Cu") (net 18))
 (segment (start 112.975 97.667) (end 103.667 97.667) (width 0.25) (layer "B.Cu") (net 18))
 (segment (start 101.000489 99.000489) (end 112.530489 99.000489) (width 0.25) (layer "F.Cu") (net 19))
 (segment (start 112.530489 99.000489) (end 112.975 99.445) (width 0.25) (layer "F.Cu") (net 19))
 (segment (start 100 98) (end 101.000489 99.000489) (width 0.25) (layer "F.Cu") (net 19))
 (segment (start 112.975 101.223) (end 105.223 101.223) (width 0.25) (layer "B.Cu") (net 20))
 (segment (start 105.223 101.223) (end 102 98) (width 0.25) (layer "B.Cu") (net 20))
 (segment (start 100.999511 100.999511) (end 110.973511 100.999511) (width 0.25) (layer "F.Cu") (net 21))
 (segment (start 110.973511 100.999511) (end 112.975 103.001) (width 0.25) (layer "F.Cu") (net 21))
 (segment (start 100 100) (end 100.999511 100.999511) (width 0.25) (layer "F.Cu") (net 21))
 (segment (start 112.975 104.779) (end 106.779 104.779) (width 0.25) (layer "B.Cu") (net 22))
 (segment (start 106.779 104.779) (end 102 100) (width 0.25) (layer "B.Cu") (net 22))
 (segment (start 100 102) (end 100.999511 102.999511) (width 0.25) (layer "F.Cu") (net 23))
 (segment (start 109.417511 102.999511) (end 112.975 106.557) (width 0.25) (layer "F.Cu") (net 23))
 (segment (start 100.999511 102.999511) (end 109.417511 102.999511) (width 0.25) (layer "F.Cu") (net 23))
 (segment (start 112.975 108.335) (end 108.335 108.335) (width 0.25) (layer "B.Cu") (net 24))
 (segment (start 108.335 108.335) (end 102 102) (width 0.25) (layer "B.Cu") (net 24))
 (segment (start 107.862489 105.000489) (end 112.975 110.113) (width 0.25) (layer "F.Cu") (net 25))
 (segment (start 100 104) (end 101.000489 105.000489) (width 0.25) (layer "F.Cu") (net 25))
 (segment (start 101.000489 105.000489) (end 107.862489 105.000489) (width 0.25) (layer "F.Cu") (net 25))
 (segment (start 112.975 111.891) (end 109.891 111.891) (width 0.25) (layer "B.Cu") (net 26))
 (segment (start 109.891 111.891) (end 102 104) (width 0.25) (layer "B.Cu") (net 26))
 (segment (start 112.975 113.669) (end 107.669 113.669) (width 0.25) (layer "F.Cu") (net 27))
 (segment (start 107.669 113.669) (end 100 106) (width 0.25) (layer "F.Cu") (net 27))
 (segment (start 112.975 115.447) (end 111.447 115.447) (width 0.25) (layer "B.Cu") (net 28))
 (segment (start 111.447 115.447) (end 102 106) (width 0.25) (layer "B.Cu") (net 28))
 (segment (start 142 77.416) (end 132.025 67.441) (width 0.25) (layer "F.Cu") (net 64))
 (segment (start 142 80) (end 142 77.416) (width 0.25) (layer "F.Cu") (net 64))
 (segment (start 133.219 69.219) (end 132.025 69.219) (width 0.25) (layer "B.Cu") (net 63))
 (segment (start 144 80) (end 133.219 69.219) (width 0.25) (layer "B.Cu") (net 63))
 (segment (start 141.000489 79.972489) (end 132.025 70.997) (width 0.25) (layer "F.Cu") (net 62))
 (segment (start 141.000489 81.000489) (end 141.000489 79.972489) (width 0.25) (layer "F.Cu") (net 62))
 (segment (start 142 82) (end 141.000489 81.000489) (width 0.25) (layer "F.Cu") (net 62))
 (segment (start 132.025 70.997) (end 132.025 71.025) (width 0.25) (layer "F.Cu") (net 62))
 (segment (start 144 82) (end 143.000489 81.000489) (width 0.25) (layer "B.Cu") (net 61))
 (segment (start 140.250489 81.000489) (end 132.025 72.775) (width 0.25) (layer "B.Cu") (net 61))
 (segment (start 143.000489 81.000489) (end 140.250489 81.000489) (width 0.25) (layer "B.Cu") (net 61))
 (segment (start 132.553 74.553) (end 132.025 74.553) (width 0.25) (layer "F.Cu") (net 60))
 (segment (start 142 84) (end 132.553 74.553) (width 0.25) (layer "F.Cu") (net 60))
 (segment (start 132.025 74.553) (end 132.025 74.623532) (width 0.25) (layer "F.Cu") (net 60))
 (segment (start 144 84) (end 142.999511 82.999511) (width 0.25) (layer "B.Cu") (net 59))
 (segment (start 142.999511 82.999511) (end 138.693511 82.999511) (width 0.25) (layer "B.Cu") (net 59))
 (segment (start 138.693511 82.999511) (end 132.025 76.331) (width 0.25) (layer "B.Cu") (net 59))
 (segment (start 142 86) (end 139.916 86) (width 0.25) (layer "F.Cu") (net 58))
 (segment (start 139.916 86) (end 132.025 78.109) (width 0.25) (layer "F.Cu") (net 58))
 (segment (start 137.137511 84.999511) (end 132.025 79.887) (width 0.25) (layer "B.Cu") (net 57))
 (segment (start 144 86) (end 142.999511 84.999511) (width 0.25) (layer "B.Cu") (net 57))
 (segment (start 142.999511 84.999511) (end 137.137511 84.999511) (width 0.25) (layer "B.Cu") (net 57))
 (segment (start 138.36 88) (end 132.025 81.665) (width 0.25) (layer "F.Cu") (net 56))
 (segment (start 142 88) (end 138.36 88) (width 0.25) (layer "F.Cu") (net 56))
 (segment (start 135.582489 87.000489) (end 132.025 83.443) (width 0.25) (layer "B.Cu") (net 55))
 (segment (start 143.000489 87.000489) (end 135.582489 87.000489) (width 0.25) (layer "B.Cu") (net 55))
 (segment (start 144 88) (end 143.000489 87.000489) (width 0.25) (layer "B.Cu") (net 55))
 (segment (start 136.804 90) (end 132.025 85.221) (width 0.25) (layer "F.Cu") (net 54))
 (segment (start 142 90) (end 136.804 90) (width 0.25) (layer "F.Cu") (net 54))
 (segment (start 134.026489 89.000489) (end 132.025 86.999) (width 0.25) (layer "B.Cu") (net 53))
 (segment (start 144 90) (end 143.000489 89.000489) (width 0.25) (layer "B.Cu") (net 53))
 (segment (start 143.000489 89.000489) (end 134.026489 89.000489) (width 0.25) (layer "B.Cu") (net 53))
 (segment (start 142 92) (end 135.177468 92) (width 0.25) (layer "F.Cu") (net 52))
 (segment (start 132.025 88.847532) (end 132.025 88.777) (width 0.25) (layer "F.Cu") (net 52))
 (segment (start 135.177468 92) (end 132.025 88.847532) (width 0.25) (layer "F.Cu") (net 52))
 (segment (start 132.470489 91.000489) (end 132.025 90.555) (width 0.25) (layer "B.Cu") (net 51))
 (segment (start 144 92) (end 143.000489 91.000489) (width 0.25) (layer "B.Cu") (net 51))
 (segment (start 143.000489 91.000489) (end 132.470489 91.000489) (width 0.25) (layer "B.Cu") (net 51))
 (segment (start 142 94) (end 141.18648 93.18648) (width 0.25) (layer "F.Cu") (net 50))
 (segment (start 132.87848 93.18648) (end 132.025 92.333) (width 0.25) (layer "F.Cu") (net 50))
 (segment (start 141.18648 93.18648) (end 132.87848 93.18648) (width 0.25) (layer "F.Cu") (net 50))
 (segment (start 143.000489 94.999511) (end 132.913511 94.999511) (width 0.25) (layer "B.Cu") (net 49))
 (segment (start 132.913511 94.999511) (end 132.025 94.111) (width 0.25) (layer "B.Cu") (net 49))
 (segment (start 144 94) (end 143.000489 94.999511) (width 0.25) (layer "B.Cu") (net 49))
 (segment (start 132.136 96) (end 132.025 95.889) (width 0.25) (layer "F.Cu") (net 48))
 (segment (start 142 96) (end 132.136 96) (width 0.25) (layer "F.Cu") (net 48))
 (segment (start 143.000489 96.999511) (end 132.692489 96.999511) (width 0.25) (layer "B.Cu") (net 47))
 (segment (start 144 96) (end 143.000489 96.999511) (width 0.25) (layer "B.Cu") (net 47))
 (segment (start 132.692489 96.999511) (end 132.025 97.667) (width 0.25) (layer "B.Cu") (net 47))
 (segment (start 140.555 99.445) (end 132.025 99.445) (width 0.25) (layer "F.Cu") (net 46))
 (segment (start 142 98) (end 140.555 99.445) (width 0.25) (layer "F.Cu") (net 46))
 (segment (start 134.248489 98.999511) (end 132.025 101.223) (width 0.25) (layer "B.Cu") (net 45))
 (segment (start 143.000489 98.999511) (end 134.248489 98.999511) (width 0.25) (layer "B.Cu") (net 45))
 (segment (start 144 98) (end 143.000489 98.999511) (width 0.25) (layer "B.Cu") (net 45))
 (segment (start 135.026 100) (end 132.025 103.001) (width 0.25) (layer "F.Cu") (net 44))
 (segment (start 142 100) (end 135.026 100) (width 0.25) (layer "F.Cu") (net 44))
 (segment (start 144 100) (end 142.999511 101.000489) (width 0.25) (layer "B.Cu") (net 43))
 (segment (start 135.803511 101.000489) (end 132.025 104.779) (width 0.25) (layer "B.Cu") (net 43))
 (segment (start 142.999511 101.000489) (end 135.803511 101.000489) (width 0.25) (layer "B.Cu") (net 43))
 (segment (start 137.443 106.557) (end 132.025 106.557) (width 0.25) (layer "F.Cu") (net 42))
 (segment (start 142 102) (end 137.443 106.557) (width 0.25) (layer "F.Cu") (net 42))
 (segment (start 142.999511 103.000489) (end 137.359511 103.000489) (width 0.25) (layer "B.Cu") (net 41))
 (segment (start 137.359511 103.000489) (end 132.025 108.335) (width 0.25) (layer "B.Cu") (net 41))
 (segment (start 144 102) (end 142.999511 103.000489) (width 0.25) (layer "B.Cu") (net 41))
 (segment (start 142 104) (end 135.887 110.113) (width 0.25) (layer "F.Cu") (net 40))
 (segment (start 135.887 110.113) (end 132.025 110.113) (width 0.25) (layer "F.Cu") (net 40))
 (segment (start 144 104) (end 143.000489 104.999511) (width 0.25) (layer "B.Cu") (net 39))
 (segment (start 138.916489 104.999511) (end 132.025 111.891) (width 0.25) (layer "B.Cu") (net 39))
 (segment (start 143.000489 104.999511) (end 138.916489 104.999511) (width 0.25) (layer "B.Cu") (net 39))
 (segment (start 134.331 113.669) (end 132.025 113.669) (width 0.25) (layer "F.Cu") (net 38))
 (segment (start 142 106) (end 134.331 113.669) (width 0.25) (layer "F.Cu") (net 38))
 (segment (start 144 106) (end 134.553 115.447) (width 0.25) (layer "B.Cu") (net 37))
 (segment (start 134.553 115.447) (end 132.025 115.447) (width 0.25) (layer "B.Cu") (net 37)))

